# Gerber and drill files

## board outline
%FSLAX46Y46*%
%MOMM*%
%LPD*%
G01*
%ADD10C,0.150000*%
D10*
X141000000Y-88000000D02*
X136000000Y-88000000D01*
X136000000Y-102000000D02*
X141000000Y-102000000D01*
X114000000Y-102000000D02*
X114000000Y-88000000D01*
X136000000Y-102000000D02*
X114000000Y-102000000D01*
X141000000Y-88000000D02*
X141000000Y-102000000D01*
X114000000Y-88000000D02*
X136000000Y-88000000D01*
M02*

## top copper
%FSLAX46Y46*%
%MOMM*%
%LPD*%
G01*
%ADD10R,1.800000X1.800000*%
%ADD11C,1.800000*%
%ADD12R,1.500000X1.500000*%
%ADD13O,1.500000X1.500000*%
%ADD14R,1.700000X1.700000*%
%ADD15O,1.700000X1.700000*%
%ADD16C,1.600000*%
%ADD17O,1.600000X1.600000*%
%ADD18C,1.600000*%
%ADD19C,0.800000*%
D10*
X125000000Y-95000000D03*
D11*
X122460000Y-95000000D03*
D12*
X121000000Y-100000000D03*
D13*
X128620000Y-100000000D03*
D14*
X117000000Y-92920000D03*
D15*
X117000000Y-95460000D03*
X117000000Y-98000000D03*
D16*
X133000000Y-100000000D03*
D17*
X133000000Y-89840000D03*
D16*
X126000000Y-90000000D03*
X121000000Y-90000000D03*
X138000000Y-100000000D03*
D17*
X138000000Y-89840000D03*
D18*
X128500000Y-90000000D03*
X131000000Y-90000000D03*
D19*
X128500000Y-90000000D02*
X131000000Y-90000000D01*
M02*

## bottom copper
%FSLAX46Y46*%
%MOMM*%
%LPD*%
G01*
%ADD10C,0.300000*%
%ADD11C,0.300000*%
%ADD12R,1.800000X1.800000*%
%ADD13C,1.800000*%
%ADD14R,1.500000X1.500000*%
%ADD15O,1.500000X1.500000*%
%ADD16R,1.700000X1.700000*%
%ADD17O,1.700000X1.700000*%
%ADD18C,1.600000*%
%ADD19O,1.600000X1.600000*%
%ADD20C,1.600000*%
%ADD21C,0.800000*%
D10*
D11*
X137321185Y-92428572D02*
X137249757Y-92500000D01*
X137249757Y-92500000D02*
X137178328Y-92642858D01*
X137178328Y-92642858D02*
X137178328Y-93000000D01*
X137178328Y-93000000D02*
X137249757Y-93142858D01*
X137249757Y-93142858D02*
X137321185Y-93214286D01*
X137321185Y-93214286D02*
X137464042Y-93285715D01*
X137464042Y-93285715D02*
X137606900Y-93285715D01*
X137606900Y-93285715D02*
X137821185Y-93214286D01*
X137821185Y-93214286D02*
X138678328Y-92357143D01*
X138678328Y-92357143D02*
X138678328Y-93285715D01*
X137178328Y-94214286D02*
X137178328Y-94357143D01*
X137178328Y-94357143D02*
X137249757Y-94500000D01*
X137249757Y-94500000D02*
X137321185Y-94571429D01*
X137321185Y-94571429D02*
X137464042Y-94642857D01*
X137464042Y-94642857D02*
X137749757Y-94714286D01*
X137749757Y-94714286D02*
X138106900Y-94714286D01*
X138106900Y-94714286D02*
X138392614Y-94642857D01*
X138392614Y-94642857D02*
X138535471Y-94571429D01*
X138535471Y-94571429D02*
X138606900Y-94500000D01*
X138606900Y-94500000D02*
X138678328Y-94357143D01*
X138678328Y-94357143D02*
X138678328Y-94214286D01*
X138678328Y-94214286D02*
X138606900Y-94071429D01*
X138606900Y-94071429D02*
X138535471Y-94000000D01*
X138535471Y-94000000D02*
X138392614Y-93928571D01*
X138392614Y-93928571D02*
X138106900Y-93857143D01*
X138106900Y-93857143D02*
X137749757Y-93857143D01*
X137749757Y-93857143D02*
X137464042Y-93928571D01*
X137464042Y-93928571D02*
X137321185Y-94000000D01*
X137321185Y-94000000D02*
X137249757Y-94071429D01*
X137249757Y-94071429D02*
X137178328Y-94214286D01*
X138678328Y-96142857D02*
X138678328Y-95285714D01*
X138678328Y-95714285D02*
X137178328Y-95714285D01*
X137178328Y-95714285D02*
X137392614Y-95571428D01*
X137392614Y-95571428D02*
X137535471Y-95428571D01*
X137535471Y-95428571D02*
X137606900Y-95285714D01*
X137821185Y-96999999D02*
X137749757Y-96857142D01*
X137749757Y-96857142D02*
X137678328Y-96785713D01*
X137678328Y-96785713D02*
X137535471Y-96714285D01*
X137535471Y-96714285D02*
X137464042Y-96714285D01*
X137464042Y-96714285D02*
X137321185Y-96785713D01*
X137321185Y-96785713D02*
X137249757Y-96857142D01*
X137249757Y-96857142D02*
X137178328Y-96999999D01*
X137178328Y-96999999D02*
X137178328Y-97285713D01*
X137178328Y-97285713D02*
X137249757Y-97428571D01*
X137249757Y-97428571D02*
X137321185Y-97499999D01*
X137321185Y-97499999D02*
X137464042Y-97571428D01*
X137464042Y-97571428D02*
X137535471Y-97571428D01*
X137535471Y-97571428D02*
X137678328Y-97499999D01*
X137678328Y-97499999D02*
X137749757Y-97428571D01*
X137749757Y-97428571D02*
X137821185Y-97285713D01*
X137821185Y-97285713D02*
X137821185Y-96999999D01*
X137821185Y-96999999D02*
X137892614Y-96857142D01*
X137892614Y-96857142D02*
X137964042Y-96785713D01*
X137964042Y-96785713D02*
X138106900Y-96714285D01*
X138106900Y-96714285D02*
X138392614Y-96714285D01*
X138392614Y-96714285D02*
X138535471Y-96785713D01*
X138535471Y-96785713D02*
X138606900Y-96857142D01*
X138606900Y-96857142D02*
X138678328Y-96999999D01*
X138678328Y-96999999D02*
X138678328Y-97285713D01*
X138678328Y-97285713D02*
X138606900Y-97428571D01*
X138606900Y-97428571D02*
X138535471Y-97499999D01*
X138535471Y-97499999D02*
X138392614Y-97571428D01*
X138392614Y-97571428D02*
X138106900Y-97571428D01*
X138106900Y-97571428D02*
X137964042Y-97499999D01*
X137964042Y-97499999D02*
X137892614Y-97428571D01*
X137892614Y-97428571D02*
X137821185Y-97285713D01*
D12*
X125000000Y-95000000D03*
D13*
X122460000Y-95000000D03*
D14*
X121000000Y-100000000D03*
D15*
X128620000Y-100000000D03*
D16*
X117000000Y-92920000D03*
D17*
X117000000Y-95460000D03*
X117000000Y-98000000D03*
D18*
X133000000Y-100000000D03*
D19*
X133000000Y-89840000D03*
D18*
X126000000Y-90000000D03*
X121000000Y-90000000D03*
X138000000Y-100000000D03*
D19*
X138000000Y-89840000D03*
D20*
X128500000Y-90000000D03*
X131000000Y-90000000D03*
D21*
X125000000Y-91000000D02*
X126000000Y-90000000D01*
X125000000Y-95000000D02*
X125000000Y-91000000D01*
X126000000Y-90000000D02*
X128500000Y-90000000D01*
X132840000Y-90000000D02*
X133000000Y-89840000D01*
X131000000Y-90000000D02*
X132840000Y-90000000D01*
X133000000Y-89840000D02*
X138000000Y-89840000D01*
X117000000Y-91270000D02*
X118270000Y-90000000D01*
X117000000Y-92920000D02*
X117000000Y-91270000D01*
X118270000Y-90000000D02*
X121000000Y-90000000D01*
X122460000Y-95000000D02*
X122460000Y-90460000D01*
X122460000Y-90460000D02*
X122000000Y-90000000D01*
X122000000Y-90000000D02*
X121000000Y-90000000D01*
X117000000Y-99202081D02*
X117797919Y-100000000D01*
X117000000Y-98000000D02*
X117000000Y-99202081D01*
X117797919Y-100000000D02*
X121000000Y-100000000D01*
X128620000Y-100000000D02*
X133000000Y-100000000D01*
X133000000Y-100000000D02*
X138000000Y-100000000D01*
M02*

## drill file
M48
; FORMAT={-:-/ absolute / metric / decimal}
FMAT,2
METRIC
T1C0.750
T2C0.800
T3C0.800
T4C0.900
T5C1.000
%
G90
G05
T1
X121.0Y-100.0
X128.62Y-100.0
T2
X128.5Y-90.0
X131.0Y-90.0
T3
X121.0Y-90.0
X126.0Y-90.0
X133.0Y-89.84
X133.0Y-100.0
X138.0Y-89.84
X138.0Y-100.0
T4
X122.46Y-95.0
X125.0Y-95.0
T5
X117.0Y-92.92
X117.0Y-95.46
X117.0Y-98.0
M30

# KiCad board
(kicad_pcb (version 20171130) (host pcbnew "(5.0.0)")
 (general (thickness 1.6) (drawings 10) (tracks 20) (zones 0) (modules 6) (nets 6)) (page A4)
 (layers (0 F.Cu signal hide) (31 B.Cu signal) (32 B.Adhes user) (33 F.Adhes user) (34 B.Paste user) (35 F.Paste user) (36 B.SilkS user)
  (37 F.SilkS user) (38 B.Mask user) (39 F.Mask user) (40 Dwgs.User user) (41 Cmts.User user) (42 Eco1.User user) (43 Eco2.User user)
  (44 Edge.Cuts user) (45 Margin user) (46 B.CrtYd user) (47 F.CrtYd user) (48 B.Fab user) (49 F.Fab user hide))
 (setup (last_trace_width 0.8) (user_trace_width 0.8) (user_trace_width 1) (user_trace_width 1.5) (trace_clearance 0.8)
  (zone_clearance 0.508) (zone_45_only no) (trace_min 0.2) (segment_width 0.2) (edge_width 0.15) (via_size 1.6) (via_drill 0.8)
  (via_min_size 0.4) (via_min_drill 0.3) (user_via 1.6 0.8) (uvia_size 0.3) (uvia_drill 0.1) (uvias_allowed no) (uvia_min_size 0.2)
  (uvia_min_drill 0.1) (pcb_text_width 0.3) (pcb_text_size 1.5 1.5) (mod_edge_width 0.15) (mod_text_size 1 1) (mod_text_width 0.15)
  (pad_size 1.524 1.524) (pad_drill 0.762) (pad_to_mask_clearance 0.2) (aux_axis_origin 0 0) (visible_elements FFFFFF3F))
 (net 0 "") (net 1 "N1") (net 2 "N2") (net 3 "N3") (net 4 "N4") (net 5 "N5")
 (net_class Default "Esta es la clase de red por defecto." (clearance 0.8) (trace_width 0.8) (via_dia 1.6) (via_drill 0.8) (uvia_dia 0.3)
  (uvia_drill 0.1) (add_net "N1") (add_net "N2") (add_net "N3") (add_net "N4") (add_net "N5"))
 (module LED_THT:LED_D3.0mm (layer F.Cu) (at 125 95 180)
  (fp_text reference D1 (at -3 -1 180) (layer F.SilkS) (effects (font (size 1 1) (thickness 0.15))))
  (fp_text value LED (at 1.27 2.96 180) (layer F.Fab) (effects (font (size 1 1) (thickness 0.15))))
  (pad 1 thru_hole rect (at 0 0 180) (size 1.8 1.8) (drill 0.9) (layers *.Cu *.Mask) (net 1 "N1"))
  (pad 2 thru_hole circle (at 2.54 0 180) (size 1.8 1.8) (drill 0.9) (layers *.Cu *.Mask) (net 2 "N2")))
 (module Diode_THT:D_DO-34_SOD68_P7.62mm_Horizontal (layer F.Cu) (at 121 100)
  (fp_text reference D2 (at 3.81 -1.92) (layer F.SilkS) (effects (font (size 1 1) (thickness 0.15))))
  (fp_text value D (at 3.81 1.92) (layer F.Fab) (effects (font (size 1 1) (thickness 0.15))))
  (pad 1 thru_hole rect (at 0 0) (size 1.5 1.5) (drill 0.75) (layers *.Cu *.Mask) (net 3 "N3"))
  (pad 2 thru_hole oval (at 7.62 0) (size 1.5 1.5) (drill 0.75) (layers *.Cu *.Mask) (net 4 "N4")))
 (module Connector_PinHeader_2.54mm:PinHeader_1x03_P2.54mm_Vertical (layer F.Cu) (at 117 92.92)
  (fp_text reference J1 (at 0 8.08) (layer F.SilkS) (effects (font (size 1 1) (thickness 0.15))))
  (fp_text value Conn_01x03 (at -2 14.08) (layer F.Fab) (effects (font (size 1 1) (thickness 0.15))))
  (pad 1 thru_hole rect (at 0 0) (size 1.7 1.7) (drill 1) (layers *.Cu *.Mask) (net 2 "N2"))
  (pad 2 thru_hole oval (at 0 2.54) (size 1.7 1.7) (drill 1) (layers *.Cu *.Mask) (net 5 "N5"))
  (pad 3 thru_hole oval (at 0 5.08) (size 1.7 1.7) (drill 1) (layers *.Cu *.Mask) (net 3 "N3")))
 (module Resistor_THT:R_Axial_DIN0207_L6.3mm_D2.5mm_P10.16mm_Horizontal (layer F.Cu) (at 133 100 90)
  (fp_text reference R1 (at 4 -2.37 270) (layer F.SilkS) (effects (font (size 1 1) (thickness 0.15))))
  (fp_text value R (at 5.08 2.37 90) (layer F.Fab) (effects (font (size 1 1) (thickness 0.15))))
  (pad 1 thru_hole circle (at 0 0 90) (size 1.6 1.6) (drill 0.8) (layers *.Cu *.Mask) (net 4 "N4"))
  (pad 2 thru_hole oval (at 10.16 0 90) (size 1.6 1.6) (drill 0.8) (layers *.Cu *.Mask) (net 1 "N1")))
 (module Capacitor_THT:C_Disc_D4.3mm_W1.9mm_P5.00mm (layer F.Cu) (at 126 90 180)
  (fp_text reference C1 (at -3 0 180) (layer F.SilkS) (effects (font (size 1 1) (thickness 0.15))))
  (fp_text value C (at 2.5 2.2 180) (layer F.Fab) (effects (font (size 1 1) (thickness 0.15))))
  (pad 1 thru_hole circle (at 0 0 180) (size 1.6 1.6) (drill 0.8) (layers *.Cu *.Mask) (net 1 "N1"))
  (pad 2 thru_hole circle (at 5 0 180) (size 1.6 1.6) (drill 0.8) (layers *.Cu *.Mask) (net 2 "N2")))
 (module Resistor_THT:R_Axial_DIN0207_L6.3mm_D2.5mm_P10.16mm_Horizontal (layer F.Cu) (at 138 100 90)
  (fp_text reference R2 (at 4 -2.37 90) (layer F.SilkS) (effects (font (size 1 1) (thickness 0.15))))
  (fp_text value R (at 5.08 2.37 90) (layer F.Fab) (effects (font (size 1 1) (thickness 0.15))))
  (pad 1 thru_hole circle (at 0 0 90) (size 1.6 1.6) (drill 0.8) (layers *.Cu *.Mask) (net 4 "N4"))
  (pad 2 thru_hole oval (at 10.16 0 90) (size 1.6 1.6) (drill 0.8) (layers *.Cu *.Mask) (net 1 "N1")))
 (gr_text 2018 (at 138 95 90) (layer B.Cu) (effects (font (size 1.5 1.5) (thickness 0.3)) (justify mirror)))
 (gr_line (start 141 88) (end 136 88) (layer Edge.Cuts) (width 0.15))
 (gr_line (start 136 102) (end 141 102) (layer Edge.Cuts) (width 0.15))
 (gr_line (start 114 102) (end 114 88) (layer Edge.Cuts) (width 0.15))
 (gr_line (start 136 102) (end 114 102) (layer Edge.Cuts) (width 0.15))
 (gr_line (start 141 88) (end 141 102) (layer Edge.Cuts) (width 0.15))
 (gr_line (start 114 88) (end 136 88) (layer Edge.Cuts) (width 0.15))
 (segment (start 125 91) (end 126 90) (width 0.8) (layer B.Cu) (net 1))
 (segment (start 125 95) (end 125 91) (width 0.8) (layer B.Cu) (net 1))
 (via (at 128.5 90) (size 1.6) (drill 0.8) (layers F.Cu B.Cu) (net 1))
 (segment (start 126 90) (end 128.5 90) (width 0.8) (layer B.Cu) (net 1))
 (via (at 131 90) (size 1.6) (drill 0.8) (layers F.Cu B.Cu) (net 1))
 (segment (start 128.5 90) (end 131 90) (width 0.8) (layer F.Cu) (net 1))
 (segment (start 132.84 90) (end 133 89.84) (width 0.8) (layer B.Cu) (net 1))
 (segment (start 131 90) (end 132.84 90) (width 0.8) (layer B.Cu) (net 1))
 (segment (start 133 89.84) (end 138 89.84) (width 0.8) (layer B.Cu) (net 1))
 (segment (start 117 91.27) (end 118.27 90) (width 0.8) (layer B.Cu) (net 2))
 (segment (start 117 92.92) (end 117 91.27) (width 0.8) (layer B.Cu) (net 2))
 (segment (start 118.27 90) (end 121 90) (width 0.8) (layer B.Cu) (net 2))
 (segment (start 122.46 95) (end 122.46 90.46) (width 0.8) (layer B.Cu) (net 2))
 (segment (start 122.46 90.46) (end 122 90) (width 0.8) (layer B.Cu) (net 2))
 (segment (start 122 90) (end 121 90) (width 0.8) (layer B.Cu) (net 2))
 (segment (start 117 99.202081) (end 117.797919 100) (width 0.8) (layer B.Cu) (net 3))
 (segment (start 117 98) (end 117 99.202081) (width 0.8) (layer B.Cu) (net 3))
 (segment (start 117.797919 100) (end 121 100) (width 0.8) (layer B.Cu) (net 3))
 (segment (start 128.62 100) (end 133 100) (width 0.8) (layer B.Cu) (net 4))
 (segment (start 133 100) (end 138 100) (width 0.8) (layer B.Cu) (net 4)))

